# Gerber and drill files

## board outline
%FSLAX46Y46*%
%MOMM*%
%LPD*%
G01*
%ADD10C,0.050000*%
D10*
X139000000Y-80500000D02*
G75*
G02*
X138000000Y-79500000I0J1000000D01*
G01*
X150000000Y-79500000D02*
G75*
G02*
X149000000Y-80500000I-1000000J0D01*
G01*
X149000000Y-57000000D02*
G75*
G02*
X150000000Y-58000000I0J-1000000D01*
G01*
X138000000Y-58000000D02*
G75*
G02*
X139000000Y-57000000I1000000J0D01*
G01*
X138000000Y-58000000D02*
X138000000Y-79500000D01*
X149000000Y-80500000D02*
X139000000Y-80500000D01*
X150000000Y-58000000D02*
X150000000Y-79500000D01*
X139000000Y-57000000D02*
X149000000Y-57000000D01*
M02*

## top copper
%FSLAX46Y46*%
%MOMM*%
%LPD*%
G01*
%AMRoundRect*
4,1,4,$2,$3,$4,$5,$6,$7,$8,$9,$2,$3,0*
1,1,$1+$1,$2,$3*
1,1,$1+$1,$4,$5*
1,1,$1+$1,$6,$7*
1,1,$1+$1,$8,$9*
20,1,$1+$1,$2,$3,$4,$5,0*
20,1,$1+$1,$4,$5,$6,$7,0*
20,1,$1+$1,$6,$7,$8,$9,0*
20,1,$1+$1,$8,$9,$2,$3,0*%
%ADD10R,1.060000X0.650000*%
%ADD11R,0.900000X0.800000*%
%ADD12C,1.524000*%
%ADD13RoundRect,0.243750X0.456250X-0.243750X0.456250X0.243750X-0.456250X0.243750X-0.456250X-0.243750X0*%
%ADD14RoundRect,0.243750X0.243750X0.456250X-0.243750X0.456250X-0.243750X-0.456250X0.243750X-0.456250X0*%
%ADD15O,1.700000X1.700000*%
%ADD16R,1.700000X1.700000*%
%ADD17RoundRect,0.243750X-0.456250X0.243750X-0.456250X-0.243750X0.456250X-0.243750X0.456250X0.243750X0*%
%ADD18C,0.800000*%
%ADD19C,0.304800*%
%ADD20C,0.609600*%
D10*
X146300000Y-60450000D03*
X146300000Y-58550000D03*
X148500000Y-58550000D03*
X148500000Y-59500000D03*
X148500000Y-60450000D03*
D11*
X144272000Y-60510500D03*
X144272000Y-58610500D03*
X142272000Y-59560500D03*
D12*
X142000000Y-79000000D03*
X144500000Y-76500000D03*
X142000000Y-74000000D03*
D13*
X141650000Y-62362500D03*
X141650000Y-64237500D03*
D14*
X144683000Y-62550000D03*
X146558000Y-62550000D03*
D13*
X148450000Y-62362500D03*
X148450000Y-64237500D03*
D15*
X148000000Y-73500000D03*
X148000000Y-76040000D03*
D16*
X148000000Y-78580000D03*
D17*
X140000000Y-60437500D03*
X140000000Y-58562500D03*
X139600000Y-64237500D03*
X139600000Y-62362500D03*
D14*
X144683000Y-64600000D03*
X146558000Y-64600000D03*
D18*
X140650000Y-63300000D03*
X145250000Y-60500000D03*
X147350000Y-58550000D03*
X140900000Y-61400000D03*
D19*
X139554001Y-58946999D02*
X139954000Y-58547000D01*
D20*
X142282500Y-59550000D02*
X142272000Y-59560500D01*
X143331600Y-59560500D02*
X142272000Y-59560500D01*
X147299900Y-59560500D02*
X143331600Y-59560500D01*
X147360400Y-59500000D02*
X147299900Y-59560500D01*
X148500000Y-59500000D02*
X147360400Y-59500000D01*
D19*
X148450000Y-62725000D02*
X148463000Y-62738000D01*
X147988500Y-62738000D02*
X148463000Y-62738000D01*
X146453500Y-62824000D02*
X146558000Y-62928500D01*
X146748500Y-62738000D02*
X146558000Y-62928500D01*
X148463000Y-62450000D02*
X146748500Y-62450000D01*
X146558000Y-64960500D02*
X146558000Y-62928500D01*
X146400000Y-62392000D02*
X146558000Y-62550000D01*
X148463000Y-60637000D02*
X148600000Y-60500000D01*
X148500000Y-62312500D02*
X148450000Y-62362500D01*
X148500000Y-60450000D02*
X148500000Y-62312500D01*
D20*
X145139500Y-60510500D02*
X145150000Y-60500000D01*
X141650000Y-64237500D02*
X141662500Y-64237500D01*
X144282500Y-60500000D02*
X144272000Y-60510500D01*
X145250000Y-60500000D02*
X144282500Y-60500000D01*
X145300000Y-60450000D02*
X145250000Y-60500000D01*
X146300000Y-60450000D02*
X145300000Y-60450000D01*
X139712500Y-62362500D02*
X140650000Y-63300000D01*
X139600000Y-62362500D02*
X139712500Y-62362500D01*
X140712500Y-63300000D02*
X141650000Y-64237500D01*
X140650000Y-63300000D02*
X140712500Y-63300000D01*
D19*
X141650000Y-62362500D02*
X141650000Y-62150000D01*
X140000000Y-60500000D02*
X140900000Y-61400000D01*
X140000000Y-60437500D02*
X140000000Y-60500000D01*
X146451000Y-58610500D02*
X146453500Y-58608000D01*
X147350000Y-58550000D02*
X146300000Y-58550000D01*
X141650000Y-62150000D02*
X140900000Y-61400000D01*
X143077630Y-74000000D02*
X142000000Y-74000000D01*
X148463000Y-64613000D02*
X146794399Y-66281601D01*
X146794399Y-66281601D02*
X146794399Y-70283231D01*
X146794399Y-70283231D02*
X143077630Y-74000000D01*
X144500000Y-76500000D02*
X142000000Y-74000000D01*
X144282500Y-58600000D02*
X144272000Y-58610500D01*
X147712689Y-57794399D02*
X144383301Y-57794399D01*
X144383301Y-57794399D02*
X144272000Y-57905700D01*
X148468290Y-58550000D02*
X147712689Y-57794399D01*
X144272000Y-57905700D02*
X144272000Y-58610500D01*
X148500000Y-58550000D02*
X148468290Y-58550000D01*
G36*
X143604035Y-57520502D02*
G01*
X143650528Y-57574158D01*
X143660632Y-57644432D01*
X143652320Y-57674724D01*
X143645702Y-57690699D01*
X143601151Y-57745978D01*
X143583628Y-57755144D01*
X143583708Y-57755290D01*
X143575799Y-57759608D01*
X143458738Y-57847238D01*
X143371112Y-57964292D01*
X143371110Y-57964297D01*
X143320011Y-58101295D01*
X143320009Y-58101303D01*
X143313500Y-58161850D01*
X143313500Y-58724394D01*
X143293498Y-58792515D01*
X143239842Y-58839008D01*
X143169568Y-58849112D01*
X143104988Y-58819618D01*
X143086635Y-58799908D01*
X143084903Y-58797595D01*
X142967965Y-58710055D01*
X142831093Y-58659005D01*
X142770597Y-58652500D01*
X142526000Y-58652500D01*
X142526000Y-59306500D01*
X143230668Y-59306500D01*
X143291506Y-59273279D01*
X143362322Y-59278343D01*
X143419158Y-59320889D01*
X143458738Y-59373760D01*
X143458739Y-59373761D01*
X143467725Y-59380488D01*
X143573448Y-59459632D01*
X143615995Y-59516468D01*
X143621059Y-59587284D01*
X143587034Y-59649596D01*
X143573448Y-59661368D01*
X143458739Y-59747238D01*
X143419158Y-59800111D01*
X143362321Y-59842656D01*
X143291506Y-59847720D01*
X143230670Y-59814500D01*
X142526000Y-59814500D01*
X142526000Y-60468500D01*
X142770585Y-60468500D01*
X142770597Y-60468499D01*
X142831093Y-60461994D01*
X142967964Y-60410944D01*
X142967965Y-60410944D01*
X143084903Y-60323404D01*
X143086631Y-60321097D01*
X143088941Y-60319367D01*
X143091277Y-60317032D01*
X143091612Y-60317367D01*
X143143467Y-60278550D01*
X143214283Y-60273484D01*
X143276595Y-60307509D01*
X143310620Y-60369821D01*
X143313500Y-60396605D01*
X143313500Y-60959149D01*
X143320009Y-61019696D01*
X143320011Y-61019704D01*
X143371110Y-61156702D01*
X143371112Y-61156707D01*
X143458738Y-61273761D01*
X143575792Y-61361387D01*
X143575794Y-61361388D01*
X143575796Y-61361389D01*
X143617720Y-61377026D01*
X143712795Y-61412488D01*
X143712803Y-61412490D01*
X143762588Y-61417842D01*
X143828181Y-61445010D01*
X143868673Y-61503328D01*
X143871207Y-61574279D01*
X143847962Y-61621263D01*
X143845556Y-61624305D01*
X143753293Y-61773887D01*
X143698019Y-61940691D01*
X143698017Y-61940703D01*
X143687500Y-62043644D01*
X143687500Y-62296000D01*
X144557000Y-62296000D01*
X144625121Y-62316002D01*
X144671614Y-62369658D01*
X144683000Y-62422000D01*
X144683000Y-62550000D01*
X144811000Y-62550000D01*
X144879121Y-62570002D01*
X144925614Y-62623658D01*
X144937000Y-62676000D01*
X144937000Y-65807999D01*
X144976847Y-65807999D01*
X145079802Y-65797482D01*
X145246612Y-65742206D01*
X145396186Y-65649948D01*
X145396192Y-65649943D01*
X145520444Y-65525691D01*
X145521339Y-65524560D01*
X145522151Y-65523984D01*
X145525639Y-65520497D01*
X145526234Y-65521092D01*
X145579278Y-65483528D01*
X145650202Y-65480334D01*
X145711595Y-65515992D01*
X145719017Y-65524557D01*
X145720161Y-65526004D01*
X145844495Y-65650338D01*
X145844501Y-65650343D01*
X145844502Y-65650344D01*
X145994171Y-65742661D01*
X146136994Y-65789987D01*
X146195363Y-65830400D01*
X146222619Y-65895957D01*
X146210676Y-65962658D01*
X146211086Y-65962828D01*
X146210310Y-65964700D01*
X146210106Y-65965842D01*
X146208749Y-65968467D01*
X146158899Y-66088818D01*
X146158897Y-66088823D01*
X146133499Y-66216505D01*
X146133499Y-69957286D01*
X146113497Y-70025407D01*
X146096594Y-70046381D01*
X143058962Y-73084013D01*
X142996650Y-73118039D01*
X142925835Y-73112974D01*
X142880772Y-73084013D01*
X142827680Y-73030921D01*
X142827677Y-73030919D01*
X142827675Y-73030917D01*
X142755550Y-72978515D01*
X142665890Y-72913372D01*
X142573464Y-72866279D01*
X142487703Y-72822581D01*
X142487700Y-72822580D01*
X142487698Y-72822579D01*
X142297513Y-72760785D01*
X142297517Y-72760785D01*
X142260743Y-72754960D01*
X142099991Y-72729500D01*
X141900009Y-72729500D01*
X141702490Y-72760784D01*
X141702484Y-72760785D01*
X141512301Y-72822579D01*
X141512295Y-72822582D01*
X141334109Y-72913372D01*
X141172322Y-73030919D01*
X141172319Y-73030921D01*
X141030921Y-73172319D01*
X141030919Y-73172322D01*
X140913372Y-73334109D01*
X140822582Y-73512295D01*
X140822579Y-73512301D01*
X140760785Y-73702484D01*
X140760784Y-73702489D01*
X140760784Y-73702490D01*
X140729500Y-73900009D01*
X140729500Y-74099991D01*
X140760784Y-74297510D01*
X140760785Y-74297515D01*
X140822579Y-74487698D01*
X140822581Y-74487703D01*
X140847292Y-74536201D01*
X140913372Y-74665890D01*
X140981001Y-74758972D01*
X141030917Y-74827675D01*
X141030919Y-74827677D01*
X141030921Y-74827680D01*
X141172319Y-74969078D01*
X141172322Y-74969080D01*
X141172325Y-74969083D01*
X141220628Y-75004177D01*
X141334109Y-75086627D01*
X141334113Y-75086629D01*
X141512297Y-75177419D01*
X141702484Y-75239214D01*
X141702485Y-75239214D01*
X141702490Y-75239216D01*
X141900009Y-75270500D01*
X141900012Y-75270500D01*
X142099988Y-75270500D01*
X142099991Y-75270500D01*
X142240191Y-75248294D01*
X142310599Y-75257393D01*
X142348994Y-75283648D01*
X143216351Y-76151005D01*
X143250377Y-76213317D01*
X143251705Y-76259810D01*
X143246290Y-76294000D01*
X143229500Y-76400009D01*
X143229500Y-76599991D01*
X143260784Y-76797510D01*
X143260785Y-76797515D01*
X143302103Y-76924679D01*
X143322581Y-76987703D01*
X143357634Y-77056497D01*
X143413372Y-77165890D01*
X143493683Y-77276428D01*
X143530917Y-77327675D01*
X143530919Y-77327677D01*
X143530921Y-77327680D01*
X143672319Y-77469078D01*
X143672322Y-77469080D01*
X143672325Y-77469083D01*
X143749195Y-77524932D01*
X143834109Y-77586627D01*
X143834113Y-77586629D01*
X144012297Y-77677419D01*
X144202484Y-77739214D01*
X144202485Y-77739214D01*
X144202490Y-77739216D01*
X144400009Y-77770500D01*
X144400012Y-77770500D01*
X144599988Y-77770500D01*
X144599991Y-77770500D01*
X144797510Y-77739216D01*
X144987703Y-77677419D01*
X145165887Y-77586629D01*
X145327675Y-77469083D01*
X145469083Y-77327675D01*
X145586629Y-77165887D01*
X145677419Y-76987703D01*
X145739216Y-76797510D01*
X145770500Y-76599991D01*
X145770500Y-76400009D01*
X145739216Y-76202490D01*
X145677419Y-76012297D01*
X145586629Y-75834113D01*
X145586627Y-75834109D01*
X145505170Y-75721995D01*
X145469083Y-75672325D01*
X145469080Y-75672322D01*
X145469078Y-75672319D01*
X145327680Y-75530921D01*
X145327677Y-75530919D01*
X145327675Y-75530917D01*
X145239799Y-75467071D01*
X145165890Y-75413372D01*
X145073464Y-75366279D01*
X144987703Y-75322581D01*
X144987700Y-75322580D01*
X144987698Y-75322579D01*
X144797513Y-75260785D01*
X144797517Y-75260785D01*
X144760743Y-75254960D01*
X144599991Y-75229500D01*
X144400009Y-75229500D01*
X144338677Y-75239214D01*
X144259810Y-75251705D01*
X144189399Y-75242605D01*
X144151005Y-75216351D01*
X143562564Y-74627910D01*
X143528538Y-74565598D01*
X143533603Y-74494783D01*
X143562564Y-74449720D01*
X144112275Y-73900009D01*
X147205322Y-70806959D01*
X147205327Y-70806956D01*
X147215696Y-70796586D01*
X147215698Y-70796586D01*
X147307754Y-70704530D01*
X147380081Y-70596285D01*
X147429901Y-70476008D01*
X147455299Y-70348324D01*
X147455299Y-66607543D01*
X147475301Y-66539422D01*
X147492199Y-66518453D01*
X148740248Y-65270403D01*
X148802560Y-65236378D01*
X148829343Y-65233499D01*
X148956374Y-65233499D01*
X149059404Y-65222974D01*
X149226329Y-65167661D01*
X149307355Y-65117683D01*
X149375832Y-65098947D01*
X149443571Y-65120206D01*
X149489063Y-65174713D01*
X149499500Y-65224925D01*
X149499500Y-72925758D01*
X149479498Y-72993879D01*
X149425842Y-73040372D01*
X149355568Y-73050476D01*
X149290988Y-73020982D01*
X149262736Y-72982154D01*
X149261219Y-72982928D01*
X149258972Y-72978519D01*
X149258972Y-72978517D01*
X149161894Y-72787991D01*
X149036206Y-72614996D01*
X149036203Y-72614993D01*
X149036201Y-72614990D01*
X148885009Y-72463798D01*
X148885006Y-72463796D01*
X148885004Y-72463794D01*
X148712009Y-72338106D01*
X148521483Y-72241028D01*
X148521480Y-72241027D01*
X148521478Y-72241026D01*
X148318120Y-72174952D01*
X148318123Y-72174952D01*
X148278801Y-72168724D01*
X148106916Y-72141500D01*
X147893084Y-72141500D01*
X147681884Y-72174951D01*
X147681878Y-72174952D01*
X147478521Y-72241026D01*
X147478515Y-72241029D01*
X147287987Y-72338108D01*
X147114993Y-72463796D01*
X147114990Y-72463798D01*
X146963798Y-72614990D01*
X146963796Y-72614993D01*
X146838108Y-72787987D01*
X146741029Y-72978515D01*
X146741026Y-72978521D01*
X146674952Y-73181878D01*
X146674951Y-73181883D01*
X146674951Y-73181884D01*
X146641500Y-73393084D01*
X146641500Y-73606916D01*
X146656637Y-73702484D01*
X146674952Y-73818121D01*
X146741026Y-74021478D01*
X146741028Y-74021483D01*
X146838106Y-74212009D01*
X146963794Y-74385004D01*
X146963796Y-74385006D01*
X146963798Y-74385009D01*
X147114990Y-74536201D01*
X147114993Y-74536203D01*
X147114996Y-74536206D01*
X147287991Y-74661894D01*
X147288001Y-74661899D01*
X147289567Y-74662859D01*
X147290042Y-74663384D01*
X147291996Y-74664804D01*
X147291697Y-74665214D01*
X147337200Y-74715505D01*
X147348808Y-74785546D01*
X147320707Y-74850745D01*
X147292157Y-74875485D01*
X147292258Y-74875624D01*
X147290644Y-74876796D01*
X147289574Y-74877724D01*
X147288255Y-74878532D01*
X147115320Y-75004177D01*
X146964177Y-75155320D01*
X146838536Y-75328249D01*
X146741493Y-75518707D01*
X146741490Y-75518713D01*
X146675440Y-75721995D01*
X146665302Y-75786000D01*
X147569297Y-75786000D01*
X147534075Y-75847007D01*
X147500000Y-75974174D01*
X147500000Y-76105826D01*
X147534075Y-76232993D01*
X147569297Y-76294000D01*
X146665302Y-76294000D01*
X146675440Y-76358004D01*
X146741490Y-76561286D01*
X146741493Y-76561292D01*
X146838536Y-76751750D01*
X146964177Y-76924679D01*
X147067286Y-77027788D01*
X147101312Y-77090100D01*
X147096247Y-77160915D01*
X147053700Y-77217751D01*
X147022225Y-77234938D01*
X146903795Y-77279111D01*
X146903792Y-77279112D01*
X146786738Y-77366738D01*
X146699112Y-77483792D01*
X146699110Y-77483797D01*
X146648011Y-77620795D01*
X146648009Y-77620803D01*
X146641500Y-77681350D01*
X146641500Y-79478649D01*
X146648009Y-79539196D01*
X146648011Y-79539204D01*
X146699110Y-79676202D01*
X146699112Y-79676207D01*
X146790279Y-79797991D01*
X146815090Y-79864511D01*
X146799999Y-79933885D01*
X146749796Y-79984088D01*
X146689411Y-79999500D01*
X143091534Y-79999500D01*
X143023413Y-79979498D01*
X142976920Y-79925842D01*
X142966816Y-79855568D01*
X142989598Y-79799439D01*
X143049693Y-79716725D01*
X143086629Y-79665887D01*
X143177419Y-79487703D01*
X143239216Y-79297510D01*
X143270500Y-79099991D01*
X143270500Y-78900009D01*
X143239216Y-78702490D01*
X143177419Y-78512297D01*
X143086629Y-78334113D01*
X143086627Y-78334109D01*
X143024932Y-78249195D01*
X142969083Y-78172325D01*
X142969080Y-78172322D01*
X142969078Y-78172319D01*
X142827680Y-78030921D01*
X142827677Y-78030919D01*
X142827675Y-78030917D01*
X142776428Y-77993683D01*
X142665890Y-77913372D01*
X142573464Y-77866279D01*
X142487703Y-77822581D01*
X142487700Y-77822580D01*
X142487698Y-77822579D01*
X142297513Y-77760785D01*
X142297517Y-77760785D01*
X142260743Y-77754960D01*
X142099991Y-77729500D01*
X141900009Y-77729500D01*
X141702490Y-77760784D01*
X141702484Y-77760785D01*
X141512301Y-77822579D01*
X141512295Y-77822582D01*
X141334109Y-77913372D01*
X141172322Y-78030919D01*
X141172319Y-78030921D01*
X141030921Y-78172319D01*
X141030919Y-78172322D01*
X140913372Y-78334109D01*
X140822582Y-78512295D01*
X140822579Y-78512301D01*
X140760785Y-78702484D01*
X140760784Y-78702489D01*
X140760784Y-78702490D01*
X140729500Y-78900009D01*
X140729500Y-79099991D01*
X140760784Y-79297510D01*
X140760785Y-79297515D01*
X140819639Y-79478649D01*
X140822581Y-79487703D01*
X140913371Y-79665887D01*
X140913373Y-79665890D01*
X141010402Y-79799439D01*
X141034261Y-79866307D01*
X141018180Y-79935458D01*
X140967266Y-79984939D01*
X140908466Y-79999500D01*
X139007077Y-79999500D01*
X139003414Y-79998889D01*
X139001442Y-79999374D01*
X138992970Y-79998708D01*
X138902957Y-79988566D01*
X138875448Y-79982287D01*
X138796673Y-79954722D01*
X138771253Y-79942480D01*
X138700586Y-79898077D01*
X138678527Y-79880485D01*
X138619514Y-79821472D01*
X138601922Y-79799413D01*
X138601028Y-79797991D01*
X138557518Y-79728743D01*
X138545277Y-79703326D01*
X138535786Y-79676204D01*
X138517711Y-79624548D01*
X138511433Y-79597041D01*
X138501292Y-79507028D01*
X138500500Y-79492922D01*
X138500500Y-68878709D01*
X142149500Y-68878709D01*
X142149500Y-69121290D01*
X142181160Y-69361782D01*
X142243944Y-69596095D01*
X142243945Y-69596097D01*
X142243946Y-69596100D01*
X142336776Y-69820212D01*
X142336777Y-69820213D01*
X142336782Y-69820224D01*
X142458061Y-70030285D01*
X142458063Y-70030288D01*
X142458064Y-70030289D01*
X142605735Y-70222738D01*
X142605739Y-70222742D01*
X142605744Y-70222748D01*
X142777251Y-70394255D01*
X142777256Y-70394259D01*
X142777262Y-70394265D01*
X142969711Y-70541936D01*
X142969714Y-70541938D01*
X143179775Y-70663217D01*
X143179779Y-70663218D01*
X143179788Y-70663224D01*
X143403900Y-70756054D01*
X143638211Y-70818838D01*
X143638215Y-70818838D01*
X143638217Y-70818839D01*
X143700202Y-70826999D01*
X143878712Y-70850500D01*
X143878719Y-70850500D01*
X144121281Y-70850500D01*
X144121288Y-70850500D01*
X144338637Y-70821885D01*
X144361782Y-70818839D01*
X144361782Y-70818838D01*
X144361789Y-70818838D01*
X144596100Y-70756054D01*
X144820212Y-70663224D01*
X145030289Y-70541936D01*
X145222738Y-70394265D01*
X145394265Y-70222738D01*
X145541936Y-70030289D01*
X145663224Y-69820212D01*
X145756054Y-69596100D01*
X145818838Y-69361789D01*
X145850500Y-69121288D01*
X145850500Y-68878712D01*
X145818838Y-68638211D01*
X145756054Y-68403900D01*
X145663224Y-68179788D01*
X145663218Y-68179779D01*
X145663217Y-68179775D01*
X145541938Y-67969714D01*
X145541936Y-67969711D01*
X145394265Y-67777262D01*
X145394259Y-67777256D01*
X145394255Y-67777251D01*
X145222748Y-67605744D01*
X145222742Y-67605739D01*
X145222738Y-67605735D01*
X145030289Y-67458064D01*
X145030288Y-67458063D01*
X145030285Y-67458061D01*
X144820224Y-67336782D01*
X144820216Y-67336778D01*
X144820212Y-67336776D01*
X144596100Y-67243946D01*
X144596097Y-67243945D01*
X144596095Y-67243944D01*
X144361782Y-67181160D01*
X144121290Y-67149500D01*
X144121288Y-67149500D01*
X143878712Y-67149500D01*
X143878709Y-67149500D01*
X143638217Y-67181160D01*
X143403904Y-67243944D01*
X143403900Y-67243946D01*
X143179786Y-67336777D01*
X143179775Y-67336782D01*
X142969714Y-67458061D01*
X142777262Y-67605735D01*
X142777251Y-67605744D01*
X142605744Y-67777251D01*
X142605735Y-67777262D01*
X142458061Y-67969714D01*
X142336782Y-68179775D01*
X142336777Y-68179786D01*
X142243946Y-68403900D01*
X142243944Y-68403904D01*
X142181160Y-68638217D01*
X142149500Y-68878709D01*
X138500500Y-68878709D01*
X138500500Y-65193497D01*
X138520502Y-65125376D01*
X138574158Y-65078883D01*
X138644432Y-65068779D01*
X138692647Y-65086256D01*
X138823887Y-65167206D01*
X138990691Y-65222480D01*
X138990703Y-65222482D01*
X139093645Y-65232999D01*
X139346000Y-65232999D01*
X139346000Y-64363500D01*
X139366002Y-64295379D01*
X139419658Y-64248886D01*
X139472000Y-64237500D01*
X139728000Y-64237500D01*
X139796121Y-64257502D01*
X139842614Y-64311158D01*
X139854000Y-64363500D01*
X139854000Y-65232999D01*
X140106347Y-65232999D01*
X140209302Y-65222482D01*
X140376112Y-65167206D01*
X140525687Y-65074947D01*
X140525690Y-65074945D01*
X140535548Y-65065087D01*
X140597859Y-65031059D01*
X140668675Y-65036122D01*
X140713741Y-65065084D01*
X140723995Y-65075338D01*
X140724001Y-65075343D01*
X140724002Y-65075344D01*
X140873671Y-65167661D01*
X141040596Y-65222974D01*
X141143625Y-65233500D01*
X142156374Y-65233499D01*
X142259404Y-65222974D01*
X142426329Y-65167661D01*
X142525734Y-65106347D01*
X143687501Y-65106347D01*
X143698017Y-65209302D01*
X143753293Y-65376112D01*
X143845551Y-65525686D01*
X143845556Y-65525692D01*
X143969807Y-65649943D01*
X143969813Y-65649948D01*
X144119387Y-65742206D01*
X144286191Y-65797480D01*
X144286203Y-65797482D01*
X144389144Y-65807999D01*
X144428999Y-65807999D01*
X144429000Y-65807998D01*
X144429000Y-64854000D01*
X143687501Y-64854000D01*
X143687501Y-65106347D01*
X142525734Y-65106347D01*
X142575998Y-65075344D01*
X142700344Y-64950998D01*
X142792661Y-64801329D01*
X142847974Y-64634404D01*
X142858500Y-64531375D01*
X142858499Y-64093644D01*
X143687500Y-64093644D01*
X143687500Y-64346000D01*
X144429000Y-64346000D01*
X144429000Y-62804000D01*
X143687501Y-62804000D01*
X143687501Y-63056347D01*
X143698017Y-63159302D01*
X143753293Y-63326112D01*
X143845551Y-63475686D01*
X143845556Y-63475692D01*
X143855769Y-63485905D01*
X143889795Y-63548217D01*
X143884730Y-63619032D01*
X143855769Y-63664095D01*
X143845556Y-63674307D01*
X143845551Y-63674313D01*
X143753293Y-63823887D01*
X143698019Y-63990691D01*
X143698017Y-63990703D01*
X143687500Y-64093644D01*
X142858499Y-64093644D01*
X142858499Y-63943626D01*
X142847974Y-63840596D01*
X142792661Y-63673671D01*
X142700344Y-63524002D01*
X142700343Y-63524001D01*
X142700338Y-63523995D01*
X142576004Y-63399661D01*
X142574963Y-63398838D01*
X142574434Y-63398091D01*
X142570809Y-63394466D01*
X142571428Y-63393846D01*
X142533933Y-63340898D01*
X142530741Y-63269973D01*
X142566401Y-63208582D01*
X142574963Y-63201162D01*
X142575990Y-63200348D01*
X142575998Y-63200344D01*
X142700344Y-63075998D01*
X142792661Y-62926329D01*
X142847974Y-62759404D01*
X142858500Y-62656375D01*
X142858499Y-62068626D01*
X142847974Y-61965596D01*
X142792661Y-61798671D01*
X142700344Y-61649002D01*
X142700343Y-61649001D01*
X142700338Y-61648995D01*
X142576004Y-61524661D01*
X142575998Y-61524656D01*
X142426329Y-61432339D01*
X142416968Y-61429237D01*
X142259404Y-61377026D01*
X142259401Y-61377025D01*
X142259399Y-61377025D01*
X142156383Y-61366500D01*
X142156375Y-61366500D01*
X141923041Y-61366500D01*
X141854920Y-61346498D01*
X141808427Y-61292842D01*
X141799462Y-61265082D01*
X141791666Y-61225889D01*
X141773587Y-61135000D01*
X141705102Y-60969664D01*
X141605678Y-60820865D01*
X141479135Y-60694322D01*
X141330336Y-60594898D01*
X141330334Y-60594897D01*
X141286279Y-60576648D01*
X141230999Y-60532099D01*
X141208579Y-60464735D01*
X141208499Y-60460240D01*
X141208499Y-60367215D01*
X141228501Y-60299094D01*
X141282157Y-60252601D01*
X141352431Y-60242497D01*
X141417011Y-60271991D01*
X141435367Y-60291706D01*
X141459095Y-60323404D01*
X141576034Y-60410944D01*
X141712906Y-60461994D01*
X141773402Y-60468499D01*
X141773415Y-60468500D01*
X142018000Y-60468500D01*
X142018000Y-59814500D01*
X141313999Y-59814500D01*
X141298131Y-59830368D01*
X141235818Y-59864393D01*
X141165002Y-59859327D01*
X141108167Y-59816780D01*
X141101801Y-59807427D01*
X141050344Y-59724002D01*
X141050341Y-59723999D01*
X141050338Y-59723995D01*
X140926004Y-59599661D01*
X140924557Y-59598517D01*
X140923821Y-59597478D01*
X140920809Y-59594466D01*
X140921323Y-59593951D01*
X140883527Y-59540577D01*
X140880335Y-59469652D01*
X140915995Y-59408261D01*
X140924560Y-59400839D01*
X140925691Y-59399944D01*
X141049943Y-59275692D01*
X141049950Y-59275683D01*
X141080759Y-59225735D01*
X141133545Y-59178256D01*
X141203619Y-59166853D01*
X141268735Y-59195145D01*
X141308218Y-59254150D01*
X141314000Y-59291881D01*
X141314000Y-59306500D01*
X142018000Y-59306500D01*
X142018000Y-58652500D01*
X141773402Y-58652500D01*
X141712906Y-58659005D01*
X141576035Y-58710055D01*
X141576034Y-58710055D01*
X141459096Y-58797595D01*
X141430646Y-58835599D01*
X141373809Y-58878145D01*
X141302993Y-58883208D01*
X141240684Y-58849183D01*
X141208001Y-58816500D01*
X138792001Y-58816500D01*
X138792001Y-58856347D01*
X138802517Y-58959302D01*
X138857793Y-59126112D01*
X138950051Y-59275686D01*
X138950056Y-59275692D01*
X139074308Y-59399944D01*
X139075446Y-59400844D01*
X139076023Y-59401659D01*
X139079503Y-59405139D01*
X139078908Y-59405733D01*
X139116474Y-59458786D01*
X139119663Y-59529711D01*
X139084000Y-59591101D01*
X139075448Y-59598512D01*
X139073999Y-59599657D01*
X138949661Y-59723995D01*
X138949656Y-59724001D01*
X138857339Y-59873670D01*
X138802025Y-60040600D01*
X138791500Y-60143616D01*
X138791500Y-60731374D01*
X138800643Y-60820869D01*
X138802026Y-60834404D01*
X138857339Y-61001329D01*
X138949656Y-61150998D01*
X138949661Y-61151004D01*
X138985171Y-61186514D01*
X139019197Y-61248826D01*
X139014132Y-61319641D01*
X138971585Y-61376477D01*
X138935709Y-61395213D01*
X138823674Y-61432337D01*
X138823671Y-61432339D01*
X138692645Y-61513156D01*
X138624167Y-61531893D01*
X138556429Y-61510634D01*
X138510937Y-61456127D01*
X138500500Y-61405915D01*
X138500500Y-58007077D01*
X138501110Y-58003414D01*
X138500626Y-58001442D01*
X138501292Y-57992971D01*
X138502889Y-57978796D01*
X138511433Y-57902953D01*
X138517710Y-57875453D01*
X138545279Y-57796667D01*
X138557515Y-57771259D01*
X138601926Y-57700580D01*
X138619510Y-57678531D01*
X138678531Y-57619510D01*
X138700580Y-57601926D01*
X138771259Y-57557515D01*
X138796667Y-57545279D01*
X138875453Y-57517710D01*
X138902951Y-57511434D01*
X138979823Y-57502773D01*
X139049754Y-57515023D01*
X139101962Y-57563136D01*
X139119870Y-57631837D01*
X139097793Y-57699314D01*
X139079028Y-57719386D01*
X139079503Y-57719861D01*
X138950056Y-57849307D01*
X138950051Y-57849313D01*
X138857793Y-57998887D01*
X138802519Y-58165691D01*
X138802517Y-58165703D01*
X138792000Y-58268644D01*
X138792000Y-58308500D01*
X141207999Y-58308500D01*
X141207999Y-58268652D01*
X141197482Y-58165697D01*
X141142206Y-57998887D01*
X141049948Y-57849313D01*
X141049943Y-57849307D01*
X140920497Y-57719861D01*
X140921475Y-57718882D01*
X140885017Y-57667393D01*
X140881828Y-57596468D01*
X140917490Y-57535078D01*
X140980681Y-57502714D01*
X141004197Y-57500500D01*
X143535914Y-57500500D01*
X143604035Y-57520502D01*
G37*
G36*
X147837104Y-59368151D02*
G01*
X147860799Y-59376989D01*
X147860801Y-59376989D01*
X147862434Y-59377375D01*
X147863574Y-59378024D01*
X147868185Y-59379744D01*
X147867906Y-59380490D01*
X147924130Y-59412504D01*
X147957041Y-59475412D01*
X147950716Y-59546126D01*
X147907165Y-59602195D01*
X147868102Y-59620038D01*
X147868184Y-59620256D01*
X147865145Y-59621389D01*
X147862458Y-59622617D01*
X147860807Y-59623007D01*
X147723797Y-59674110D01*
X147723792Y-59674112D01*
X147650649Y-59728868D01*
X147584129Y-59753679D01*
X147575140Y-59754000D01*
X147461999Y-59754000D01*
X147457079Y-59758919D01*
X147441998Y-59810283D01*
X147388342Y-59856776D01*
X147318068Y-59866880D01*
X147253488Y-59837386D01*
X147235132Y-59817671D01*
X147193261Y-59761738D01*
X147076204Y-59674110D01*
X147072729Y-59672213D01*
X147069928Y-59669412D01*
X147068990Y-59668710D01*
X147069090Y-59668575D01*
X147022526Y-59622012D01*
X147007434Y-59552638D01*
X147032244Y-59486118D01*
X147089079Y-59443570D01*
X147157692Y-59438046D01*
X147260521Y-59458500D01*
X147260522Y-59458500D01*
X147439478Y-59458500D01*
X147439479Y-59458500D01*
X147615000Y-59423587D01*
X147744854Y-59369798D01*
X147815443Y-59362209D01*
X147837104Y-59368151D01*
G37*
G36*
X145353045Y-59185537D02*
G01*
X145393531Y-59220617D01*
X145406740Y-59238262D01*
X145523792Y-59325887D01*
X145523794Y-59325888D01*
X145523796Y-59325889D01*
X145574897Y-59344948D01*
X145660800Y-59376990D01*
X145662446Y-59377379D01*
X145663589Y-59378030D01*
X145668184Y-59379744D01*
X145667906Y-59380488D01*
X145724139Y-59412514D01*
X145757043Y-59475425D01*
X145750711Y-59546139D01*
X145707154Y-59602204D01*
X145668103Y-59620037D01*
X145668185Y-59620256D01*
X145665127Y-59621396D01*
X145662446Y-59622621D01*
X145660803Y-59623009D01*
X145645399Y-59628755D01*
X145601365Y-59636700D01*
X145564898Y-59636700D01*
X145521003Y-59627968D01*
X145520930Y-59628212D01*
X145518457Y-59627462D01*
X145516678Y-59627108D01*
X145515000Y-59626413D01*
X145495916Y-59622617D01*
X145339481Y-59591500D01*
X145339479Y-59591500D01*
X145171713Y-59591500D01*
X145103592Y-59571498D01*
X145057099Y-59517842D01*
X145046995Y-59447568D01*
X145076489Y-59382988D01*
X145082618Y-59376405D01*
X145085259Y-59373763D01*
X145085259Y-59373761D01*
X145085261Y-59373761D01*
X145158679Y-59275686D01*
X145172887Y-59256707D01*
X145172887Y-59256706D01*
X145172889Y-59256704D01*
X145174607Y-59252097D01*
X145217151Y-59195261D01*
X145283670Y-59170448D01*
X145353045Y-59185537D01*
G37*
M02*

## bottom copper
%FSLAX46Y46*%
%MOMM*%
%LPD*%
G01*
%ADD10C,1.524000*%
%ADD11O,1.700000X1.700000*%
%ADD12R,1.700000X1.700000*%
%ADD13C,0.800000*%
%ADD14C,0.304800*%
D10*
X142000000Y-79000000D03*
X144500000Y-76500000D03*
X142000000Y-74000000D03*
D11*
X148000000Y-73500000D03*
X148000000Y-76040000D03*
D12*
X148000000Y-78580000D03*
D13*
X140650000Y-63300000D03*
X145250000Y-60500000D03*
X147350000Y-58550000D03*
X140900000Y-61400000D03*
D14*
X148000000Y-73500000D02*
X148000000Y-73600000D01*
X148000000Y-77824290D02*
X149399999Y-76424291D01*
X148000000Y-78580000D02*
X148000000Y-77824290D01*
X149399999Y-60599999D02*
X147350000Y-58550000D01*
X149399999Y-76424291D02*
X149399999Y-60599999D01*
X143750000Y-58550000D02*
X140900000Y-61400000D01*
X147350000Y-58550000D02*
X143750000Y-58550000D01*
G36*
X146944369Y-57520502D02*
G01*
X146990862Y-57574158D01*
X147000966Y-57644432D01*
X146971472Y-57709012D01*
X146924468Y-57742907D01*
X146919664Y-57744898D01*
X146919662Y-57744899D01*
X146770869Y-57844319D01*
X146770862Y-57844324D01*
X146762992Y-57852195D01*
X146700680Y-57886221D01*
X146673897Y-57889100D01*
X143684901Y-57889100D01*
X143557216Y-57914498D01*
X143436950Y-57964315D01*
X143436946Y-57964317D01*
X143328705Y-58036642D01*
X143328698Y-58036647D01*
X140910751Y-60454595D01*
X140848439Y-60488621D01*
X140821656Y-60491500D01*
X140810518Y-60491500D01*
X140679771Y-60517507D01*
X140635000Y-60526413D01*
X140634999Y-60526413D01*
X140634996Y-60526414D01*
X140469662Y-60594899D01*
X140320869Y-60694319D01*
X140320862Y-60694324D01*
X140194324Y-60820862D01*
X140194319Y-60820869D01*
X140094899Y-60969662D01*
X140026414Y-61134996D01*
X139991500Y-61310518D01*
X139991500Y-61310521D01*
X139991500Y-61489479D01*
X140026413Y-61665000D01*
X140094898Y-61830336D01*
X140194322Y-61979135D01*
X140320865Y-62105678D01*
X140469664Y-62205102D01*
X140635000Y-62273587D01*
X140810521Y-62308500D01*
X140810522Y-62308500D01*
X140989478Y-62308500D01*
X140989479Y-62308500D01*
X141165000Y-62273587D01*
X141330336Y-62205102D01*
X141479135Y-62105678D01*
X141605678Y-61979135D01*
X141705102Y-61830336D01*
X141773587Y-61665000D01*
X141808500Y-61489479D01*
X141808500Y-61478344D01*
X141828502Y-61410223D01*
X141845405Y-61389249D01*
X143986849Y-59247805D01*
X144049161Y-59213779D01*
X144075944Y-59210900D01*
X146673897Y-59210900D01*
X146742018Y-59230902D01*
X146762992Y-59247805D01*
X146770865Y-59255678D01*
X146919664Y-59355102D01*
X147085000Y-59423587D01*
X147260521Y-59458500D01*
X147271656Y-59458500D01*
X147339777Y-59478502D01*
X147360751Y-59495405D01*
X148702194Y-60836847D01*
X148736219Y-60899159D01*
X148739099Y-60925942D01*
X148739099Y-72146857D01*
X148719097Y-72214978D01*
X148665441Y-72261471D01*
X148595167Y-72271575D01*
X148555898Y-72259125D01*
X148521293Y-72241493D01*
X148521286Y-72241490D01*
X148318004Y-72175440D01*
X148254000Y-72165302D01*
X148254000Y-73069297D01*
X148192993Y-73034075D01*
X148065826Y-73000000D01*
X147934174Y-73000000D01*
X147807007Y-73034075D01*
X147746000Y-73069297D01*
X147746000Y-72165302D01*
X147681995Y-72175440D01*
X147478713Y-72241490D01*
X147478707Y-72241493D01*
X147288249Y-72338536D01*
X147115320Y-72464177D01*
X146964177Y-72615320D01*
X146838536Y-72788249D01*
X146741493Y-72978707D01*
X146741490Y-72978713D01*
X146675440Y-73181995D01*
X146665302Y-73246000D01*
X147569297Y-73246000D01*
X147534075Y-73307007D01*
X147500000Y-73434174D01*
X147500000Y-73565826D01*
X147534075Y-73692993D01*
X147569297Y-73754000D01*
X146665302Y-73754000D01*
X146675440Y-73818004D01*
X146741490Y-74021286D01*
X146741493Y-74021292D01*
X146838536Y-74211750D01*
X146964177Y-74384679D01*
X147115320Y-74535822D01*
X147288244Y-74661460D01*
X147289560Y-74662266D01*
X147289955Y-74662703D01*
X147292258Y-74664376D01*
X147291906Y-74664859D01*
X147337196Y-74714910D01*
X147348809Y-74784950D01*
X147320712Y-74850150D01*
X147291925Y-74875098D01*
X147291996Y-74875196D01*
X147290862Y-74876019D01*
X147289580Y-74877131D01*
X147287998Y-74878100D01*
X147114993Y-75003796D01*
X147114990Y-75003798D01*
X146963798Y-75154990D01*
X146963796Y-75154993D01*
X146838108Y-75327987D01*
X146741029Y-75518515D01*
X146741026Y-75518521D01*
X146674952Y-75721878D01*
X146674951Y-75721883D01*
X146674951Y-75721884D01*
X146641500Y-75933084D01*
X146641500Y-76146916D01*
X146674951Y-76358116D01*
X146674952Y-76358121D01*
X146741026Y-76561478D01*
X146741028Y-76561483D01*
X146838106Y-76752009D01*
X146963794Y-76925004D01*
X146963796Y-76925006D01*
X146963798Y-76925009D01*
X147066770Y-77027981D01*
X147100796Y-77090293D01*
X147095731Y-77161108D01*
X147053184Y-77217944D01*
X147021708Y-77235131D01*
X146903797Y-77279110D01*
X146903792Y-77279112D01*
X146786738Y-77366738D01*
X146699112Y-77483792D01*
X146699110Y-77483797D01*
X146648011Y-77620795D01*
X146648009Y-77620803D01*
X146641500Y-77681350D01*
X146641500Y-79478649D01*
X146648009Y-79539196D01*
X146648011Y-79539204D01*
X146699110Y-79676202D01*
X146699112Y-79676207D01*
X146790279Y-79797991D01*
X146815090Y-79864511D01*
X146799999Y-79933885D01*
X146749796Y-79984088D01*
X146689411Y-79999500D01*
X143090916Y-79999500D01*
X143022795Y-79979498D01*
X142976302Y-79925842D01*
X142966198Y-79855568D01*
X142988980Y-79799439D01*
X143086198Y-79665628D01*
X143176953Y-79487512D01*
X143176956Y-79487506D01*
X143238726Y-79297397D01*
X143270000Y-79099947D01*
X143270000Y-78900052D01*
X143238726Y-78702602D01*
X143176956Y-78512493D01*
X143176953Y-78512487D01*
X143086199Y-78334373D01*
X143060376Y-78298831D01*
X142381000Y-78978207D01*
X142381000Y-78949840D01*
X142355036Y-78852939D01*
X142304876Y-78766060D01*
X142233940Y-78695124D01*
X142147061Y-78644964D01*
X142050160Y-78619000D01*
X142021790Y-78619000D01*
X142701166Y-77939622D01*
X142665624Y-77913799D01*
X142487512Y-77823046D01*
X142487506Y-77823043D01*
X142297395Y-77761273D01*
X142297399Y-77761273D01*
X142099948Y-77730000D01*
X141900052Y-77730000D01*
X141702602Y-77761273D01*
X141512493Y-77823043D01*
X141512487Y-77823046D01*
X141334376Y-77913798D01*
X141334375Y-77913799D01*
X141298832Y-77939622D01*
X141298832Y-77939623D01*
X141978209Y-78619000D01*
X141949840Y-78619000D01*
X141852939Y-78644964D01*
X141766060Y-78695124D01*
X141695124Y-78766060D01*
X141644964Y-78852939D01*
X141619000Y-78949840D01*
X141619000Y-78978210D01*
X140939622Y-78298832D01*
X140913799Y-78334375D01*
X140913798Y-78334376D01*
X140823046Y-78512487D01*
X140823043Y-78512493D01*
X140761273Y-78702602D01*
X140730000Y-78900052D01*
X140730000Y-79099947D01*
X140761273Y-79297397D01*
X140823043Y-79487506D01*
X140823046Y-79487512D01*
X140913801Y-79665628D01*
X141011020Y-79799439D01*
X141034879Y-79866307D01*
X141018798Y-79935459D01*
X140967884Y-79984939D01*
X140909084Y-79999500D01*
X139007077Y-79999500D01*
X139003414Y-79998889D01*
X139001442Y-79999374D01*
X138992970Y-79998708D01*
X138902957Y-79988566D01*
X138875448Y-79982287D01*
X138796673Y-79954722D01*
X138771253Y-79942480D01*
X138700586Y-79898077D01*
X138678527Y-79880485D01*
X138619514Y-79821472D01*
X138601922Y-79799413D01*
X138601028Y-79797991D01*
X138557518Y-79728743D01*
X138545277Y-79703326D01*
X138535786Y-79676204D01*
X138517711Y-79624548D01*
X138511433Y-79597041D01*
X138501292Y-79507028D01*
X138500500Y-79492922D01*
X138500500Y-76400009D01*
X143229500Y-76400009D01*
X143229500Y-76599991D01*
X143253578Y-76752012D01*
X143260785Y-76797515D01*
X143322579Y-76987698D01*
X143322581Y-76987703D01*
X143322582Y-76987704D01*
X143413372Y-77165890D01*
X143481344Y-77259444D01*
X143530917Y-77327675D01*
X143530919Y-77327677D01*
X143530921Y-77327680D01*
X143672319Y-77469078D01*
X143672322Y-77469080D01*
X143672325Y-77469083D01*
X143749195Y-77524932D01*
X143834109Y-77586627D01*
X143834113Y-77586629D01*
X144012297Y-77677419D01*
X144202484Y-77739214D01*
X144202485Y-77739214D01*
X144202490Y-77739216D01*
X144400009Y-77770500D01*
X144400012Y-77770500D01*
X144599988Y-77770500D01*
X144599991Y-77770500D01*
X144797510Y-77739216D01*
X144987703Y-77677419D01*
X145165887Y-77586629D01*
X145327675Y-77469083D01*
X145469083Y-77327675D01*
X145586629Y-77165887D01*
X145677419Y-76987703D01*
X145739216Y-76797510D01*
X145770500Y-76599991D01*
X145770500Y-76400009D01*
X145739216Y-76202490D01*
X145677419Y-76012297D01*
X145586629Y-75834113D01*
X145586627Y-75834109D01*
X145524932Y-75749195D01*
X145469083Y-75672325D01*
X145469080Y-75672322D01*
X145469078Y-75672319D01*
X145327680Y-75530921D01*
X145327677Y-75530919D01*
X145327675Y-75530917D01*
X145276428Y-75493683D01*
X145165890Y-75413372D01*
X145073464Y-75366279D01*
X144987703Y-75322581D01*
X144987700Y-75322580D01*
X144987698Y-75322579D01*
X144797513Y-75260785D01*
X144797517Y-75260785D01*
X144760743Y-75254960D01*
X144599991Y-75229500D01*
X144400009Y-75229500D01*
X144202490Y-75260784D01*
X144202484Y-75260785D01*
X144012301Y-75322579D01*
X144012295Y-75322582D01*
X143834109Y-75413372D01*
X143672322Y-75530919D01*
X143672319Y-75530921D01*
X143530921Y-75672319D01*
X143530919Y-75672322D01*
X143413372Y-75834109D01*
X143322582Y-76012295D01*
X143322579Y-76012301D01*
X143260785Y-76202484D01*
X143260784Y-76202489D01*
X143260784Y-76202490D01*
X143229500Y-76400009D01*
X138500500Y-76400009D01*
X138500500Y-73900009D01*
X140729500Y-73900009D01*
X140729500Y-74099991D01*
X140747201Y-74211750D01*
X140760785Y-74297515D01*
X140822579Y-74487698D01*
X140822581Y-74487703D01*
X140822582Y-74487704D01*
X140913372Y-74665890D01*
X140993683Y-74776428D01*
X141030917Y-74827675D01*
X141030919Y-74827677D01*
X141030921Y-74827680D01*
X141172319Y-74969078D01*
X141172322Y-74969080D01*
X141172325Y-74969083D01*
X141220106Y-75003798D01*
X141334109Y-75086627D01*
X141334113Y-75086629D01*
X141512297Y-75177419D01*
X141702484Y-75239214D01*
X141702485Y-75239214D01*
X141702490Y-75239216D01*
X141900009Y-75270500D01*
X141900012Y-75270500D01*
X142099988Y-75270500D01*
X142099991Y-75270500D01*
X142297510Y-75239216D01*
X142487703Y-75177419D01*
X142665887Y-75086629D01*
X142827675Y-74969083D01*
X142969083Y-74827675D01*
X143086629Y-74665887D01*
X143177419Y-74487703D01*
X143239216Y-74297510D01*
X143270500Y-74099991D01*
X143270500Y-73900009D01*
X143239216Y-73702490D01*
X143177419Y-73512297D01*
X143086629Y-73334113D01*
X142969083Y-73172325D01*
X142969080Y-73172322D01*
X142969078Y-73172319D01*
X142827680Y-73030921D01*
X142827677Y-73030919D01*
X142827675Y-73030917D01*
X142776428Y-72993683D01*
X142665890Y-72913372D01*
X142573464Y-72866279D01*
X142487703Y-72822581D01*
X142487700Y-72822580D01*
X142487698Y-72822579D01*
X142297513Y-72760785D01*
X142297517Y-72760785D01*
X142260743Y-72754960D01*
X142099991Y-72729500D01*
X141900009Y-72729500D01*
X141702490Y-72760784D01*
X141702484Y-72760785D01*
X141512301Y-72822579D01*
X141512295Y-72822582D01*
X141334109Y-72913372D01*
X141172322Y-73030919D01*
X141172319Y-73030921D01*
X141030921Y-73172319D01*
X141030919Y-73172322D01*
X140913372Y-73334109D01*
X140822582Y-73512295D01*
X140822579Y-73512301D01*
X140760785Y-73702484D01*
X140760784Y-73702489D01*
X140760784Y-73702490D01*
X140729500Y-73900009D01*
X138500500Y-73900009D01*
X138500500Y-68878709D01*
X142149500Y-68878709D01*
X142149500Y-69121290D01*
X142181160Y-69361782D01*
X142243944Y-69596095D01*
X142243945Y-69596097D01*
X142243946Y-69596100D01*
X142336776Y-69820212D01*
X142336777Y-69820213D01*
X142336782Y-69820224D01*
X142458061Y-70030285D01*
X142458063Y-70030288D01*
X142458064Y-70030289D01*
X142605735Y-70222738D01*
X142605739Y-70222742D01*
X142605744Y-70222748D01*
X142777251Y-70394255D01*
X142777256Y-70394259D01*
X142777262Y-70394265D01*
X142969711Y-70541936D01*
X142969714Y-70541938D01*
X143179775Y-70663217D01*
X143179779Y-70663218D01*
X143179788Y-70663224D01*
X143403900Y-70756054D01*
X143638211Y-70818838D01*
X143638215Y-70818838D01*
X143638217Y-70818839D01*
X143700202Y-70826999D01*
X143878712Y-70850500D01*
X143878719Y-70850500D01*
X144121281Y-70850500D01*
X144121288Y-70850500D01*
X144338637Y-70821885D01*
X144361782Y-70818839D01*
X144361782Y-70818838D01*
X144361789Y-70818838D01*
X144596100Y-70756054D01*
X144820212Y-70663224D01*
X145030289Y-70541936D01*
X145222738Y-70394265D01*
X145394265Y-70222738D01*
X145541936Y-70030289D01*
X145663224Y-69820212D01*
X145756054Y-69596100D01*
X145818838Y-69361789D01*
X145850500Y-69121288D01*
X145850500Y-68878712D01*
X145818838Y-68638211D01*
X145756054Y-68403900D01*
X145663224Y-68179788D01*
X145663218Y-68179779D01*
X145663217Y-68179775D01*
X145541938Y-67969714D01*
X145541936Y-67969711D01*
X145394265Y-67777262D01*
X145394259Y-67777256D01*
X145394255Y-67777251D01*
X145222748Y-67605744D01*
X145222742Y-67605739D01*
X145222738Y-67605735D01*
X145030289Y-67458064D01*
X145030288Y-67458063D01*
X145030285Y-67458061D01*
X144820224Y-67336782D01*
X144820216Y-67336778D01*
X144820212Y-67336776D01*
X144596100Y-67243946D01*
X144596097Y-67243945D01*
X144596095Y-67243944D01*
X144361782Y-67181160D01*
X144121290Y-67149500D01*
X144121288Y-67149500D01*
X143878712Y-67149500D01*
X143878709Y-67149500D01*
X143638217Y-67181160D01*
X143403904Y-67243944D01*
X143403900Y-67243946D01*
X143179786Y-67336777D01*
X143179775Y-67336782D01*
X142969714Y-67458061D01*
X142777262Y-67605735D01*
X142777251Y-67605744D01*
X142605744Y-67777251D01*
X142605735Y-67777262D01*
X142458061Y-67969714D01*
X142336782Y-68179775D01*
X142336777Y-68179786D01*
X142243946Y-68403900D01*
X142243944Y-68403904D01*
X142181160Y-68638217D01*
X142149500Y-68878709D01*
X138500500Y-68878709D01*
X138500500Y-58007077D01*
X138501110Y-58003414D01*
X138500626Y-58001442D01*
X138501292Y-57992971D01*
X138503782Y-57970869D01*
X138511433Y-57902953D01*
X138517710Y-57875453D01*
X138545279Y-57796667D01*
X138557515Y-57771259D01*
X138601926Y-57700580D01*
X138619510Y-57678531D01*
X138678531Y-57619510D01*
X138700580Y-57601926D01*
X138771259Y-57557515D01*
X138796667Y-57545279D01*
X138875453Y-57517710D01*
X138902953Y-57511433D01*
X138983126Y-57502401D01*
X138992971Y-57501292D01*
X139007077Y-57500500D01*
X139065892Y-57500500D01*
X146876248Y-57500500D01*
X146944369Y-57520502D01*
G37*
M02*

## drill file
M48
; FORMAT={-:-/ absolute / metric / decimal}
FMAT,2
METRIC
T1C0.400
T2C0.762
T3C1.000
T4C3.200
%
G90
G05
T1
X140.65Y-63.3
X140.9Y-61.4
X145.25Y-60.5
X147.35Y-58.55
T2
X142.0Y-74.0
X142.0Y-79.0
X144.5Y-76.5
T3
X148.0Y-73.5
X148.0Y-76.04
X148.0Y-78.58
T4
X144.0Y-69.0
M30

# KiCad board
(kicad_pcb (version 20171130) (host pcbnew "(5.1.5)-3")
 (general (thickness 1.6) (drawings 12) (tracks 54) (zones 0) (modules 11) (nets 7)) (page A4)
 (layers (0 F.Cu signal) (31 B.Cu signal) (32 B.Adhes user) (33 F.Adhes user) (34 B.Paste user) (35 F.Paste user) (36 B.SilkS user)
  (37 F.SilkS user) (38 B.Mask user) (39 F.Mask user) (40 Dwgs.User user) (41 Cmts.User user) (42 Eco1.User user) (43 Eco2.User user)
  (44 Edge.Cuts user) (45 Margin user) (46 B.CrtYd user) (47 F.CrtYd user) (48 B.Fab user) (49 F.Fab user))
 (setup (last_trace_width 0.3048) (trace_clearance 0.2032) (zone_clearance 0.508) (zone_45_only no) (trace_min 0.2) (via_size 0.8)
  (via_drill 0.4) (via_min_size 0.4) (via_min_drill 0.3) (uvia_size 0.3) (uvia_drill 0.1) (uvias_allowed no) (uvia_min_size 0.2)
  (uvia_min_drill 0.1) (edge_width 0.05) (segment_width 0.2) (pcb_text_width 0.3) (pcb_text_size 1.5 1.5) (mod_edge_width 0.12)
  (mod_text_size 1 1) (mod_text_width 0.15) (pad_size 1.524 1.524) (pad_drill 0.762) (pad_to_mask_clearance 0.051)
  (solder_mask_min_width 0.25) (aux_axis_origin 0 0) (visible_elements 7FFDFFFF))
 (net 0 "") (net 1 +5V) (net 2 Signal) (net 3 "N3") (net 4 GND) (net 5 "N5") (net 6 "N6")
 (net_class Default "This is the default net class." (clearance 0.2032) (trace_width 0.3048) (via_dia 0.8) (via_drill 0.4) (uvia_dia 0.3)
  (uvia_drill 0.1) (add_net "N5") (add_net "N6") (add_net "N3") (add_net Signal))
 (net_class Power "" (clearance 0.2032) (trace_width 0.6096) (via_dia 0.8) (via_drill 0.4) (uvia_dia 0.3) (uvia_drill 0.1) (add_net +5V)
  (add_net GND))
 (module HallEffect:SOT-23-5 (layer F.Cu) (at 147.4 59.5 180)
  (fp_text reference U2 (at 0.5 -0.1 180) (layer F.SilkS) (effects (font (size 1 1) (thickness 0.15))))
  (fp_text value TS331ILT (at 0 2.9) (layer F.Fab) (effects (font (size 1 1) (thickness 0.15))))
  (pad 5 smd rect (at 1.1 -0.95 180) (size 1.06 0.65) (layers F.Cu F.Paste F.Mask) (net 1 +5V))
  (pad 4 smd rect (at 1.1 0.95 180) (size 1.06 0.65) (layers F.Cu F.Paste F.Mask) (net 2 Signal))
  (pad 3 smd rect (at -1.1 0.95 180) (size 1.06 0.65) (layers F.Cu F.Paste F.Mask) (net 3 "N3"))
  (pad 2 smd rect (at -1.1 0 180) (size 1.06 0.65) (layers F.Cu F.Paste F.Mask) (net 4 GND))
  (pad 1 smd rect (at -1.1 -0.95 180) (size 1.06 0.65) (layers F.Cu F.Paste F.Mask) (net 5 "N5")))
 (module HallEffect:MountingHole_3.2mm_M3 (layer F.Cu) (at 144 69)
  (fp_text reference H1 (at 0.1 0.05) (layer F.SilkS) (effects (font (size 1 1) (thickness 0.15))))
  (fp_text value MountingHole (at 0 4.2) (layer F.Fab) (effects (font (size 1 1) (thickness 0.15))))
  (pad 1 np_thru_hole circle (at 0 0) (size 3.2 3.2) (drill 3.2) (layers *.Cu *.Mask)))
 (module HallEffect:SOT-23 (layer F.Cu) (at 143.272 59.5605 180)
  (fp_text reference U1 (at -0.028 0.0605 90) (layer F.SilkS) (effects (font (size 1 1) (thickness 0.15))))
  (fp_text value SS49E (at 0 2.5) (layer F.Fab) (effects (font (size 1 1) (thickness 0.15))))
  (pad 1 smd rect (at -1 -0.95 180) (size 0.9 0.8) (layers F.Cu F.Paste F.Mask) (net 1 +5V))
  (pad 2 smd rect (at -1 0.95 180) (size 0.9 0.8) (layers F.Cu F.Paste F.Mask) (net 3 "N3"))
  (pad 3 smd rect (at 1 0 180) (size 0.9 0.8) (layers F.Cu F.Paste F.Mask) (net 4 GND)))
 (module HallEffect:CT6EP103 (layer F.Cu) (at 142 76.5 270)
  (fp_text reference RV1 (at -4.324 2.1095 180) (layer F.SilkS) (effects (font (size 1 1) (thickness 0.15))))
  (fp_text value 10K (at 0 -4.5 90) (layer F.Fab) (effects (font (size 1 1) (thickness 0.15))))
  (pad 3 thru_hole circle (at 2.5 0 270) (size 1.524 1.524) (drill 0.762) (layers *.Cu *.Mask) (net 1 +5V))
  (pad 2 thru_hole circle (at 0 -2.5 270) (size 1.524 1.524) (drill 0.762) (layers *.Cu *.Mask) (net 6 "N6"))
  (pad 1 thru_hole circle (at -2.5 0 270) (size 1.524 1.524) (drill 0.762) (layers *.Cu *.Mask) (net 6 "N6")))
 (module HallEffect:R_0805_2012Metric (layer F.Cu) (at 141.65 63.3 90)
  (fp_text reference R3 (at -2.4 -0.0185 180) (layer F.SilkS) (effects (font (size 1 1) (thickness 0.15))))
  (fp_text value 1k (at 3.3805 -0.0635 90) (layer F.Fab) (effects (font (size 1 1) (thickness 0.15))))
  (pad 2 smd roundrect (at 0.9375 0 90) (size 0.975 1.4) (layers F.Cu F.Paste F.Mask) (roundrect_rratio 0.25) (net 2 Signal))
  (pad 1 smd roundrect (at -0.9375 0 90) (size 0.975 1.4) (layers F.Cu F.Paste F.Mask) (roundrect_rratio 0.25) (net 1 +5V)))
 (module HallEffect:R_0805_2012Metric (layer F.Cu) (at 145.6205 62.55 180)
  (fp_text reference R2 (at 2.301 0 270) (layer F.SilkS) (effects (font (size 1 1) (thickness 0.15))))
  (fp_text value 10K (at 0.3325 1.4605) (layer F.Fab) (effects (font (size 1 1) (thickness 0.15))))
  (pad 2 smd roundrect (at 0.9375 0 180) (size 0.975 1.4) (layers F.Cu F.Paste F.Mask) (roundrect_rratio 0.25) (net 4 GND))
  (pad 1 smd roundrect (at -0.9375 0 180) (size 0.975 1.4) (layers F.Cu F.Paste F.Mask) (roundrect_rratio 0.25) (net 5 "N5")))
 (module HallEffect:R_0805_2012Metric (layer F.Cu) (at 148.45 63.3 90)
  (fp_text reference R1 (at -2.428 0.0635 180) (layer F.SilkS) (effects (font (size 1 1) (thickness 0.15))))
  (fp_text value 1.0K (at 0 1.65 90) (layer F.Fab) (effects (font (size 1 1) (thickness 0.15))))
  (pad 2 smd roundrect (at 0.9375 0 90) (size 0.975 1.4) (layers F.Cu F.Paste F.Mask) (roundrect_rratio 0.25) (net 5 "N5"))
  (pad 1 smd roundrect (at -0.9375 0 90) (size 0.975 1.4) (layers F.Cu F.Paste F.Mask) (roundrect_rratio 0.25) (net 6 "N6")))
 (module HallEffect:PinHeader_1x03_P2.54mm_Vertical (layer F.Cu) (at 148 78.58 180)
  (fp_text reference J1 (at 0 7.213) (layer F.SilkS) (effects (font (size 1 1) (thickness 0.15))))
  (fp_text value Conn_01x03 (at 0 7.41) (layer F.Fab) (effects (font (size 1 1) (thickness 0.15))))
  (pad 3 thru_hole oval (at 0 5.08 180) (size 1.7 1.7) (drill 1) (layers *.Cu *.Mask) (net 1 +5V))
  (pad 2 thru_hole oval (at 0 2.54 180) (size 1.7 1.7) (drill 1) (layers *.Cu *.Mask) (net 4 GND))
  (pad 1 thru_hole rect (at 0 0 180) (size 1.7 1.7) (drill 1) (layers *.Cu *.Mask) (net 2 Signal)))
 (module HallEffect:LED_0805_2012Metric (layer F.Cu) (at 140 59.5 270)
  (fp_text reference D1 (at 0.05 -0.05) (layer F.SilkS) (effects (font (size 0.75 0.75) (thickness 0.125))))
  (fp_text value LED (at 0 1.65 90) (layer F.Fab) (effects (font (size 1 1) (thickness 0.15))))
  (pad 2 smd roundrect (at 0.9375 0 270) (size 0.975 1.4) (layers F.Cu F.Paste F.Mask) (roundrect_rratio 0.25) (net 2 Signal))
  (pad 1 smd roundrect (at -0.9375 0 270) (size 0.975 1.4) (layers F.Cu F.Paste F.Mask) (roundrect_rratio 0.25) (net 4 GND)))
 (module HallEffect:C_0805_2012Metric (layer F.Cu) (at 139.6 63.3 270)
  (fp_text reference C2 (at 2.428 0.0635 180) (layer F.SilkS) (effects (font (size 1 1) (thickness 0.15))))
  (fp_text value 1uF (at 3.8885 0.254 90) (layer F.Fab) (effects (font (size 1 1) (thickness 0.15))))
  (pad 2 smd roundrect (at 0.9375 0 270) (size 0.975 1.4) (layers F.Cu F.Paste F.Mask) (roundrect_rratio 0.25) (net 4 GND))
  (pad 1 smd roundrect (at -0.9375 0 270) (size 0.975 1.4) (layers F.Cu F.Paste F.Mask) (roundrect_rratio 0.25) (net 1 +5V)))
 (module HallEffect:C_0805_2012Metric (layer F.Cu) (at 145.6205 64.6 180)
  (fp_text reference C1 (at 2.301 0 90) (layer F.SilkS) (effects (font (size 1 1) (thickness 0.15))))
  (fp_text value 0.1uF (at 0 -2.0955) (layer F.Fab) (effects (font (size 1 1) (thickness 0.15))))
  (pad 2 smd roundrect (at 0.9375 0 180) (size 0.975 1.4) (layers F.Cu F.Paste F.Mask) (roundrect_rratio 0.25) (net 4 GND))
  (pad 1 smd roundrect (at -0.9375 0 180) (size 0.975 1.4) (layers F.Cu F.Paste F.Mask) (roundrect_rratio 0.25) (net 5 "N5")))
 (gr_arc (start 139 79.5) (end 138 79.5) (angle -90) (layer Edge.Cuts) (width 0.05))
 (gr_arc (start 149 79.5) (end 149 80.5) (angle -90) (layer Edge.Cuts) (width 0.05))
 (gr_arc (start 149 58) (end 150 58) (angle -90) (layer Edge.Cuts) (width 0.05))
 (gr_arc (start 139 58) (end 139 57) (angle -90) (layer Edge.Cuts) (width 0.05))
 (gr_line (start 138 58) (end 138 79.5) (layer Edge.Cuts) (width 0.05))
 (gr_line (start 149 80.5) (end 139 80.5) (layer Edge.Cuts) (width 0.05))
 (gr_line (start 150 58) (end 150 79.5) (layer Edge.Cuts) (width 0.05))
 (gr_line (start 139 57) (end 149 57) (layer Edge.Cuts) (width 0.05))
 (segment (start 139.554001 58.946999) (end 139.954 58.547) (width 0.3048) (layer F.Cu) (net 4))
 (segment (start 142.2825 59.55) (end 142.272 59.5605) (width 0.6096) (layer F.Cu) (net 4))
 (segment (start 143.3316 59.5605) (end 142.272 59.5605) (width 0.6096) (layer F.Cu) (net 4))
 (segment (start 147.2999 59.5605) (end 143.3316 59.5605) (width 0.6096) (layer F.Cu) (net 4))
 (segment (start 147.3604 59.5) (end 147.2999 59.5605) (width 0.6096) (layer F.Cu) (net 4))
 (segment (start 148.5 59.5) (end 147.3604 59.5) (width 0.6096) (layer F.Cu) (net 4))
 (segment (start 148.45 62.725) (end 148.463 62.738) (width 0.3048) (layer F.Cu) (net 5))
 (segment (start 147.9885 62.738) (end 148.463 62.738) (width 0.3048) (layer F.Cu) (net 5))
 (segment (start 146.4535 62.824) (end 146.558 62.9285) (width 0.3048) (layer F.Cu) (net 5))
 (segment (start 146.7485 62.738) (end 146.558 62.9285) (width 0.3048) (layer F.Cu) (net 5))
 (segment (start 148.463 62.45) (end 146.7485 62.45) (width 0.3048) (layer F.Cu) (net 5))
 (segment (start 146.558 64.9605) (end 146.558 62.9285) (width 0.3048) (layer F.Cu) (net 5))
 (segment (start 146.4 62.392) (end 146.558 62.55) (width 0.3048) (layer F.Cu) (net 5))
 (segment (start 148.463 60.637) (end 148.6 60.5) (width 0.3048) (layer F.Cu) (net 5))
 (segment (start 148.5 62.3125) (end 148.45 62.3625) (width 0.3048) (layer F.Cu) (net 5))
 (segment (start 148.5 60.45) (end 148.5 62.3125) (width 0.3048) (layer F.Cu) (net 5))
 (via (at 140.65 63.3) (size 0.8) (drill 0.4) (layers F.Cu B.Cu) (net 1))
 (via (at 145.25 60.5) (size 0.8) (drill 0.4) (layers F.Cu B.Cu) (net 1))
 (segment (start 145.1395 60.5105) (end 145.15 60.5) (width 0.6096) (layer F.Cu) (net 1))
 (segment (start 141.65 64.2375) (end 141.6625 64.2375) (width 0.6096) (layer F.Cu) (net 1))
 (segment (start 148 73.5) (end 148 73.6) (width 0.3048) (layer B.Cu) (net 1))
 (segment (start 144.2825 60.5) (end 144.272 60.5105) (width 0.6096) (layer F.Cu) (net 1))
 (segment (start 145.25 60.5) (end 144.2825 60.5) (width 0.6096) (layer F.Cu) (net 1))
 (segment (start 145.3 60.45) (end 145.25 60.5) (width 0.6096) (layer F.Cu) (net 1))
 (segment (start 146.3 60.45) (end 145.3 60.45) (width 0.6096) (layer F.Cu) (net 1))
 (segment (start 139.7125 62.3625) (end 140.65 63.3) (width 0.6096) (layer F.Cu) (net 1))
 (segment (start 139.6 62.3625) (end 139.7125 62.3625) (width 0.6096) (layer F.Cu) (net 1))
 (segment (start 140.7125 63.3) (end 141.65 64.2375) (width 0.6096) (layer F.Cu) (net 1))
 (segment (start 140.65 63.3) (end 140.7125 63.3) (width 0.6096) (layer F.Cu) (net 1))
 (via (at 147.35 58.55) (size 0.8) (drill 0.4) (layers F.Cu B.Cu) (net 2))
 (via (at 140.9 61.4) (size 0.8) (drill 0.4) (layers F.Cu B.Cu) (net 2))
 (segment (start 141.65 62.3625) (end 141.65 62.15) (width 0.3048) (layer F.Cu) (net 2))
 (segment (start 140 60.5) (end 140.9 61.4) (width 0.3048) (layer F.Cu) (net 2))
 (segment (start 140 60.4375) (end 140 60.5) (width 0.3048) (layer F.Cu) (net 2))
 (segment (start 148 77.82429) (end 149.399999 76.424291) (width 0.3048) (layer B.Cu) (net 2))
 (segment (start 148 78.58) (end 148 77.82429) (width 0.3048) (layer B.Cu) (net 2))
 (segment (start 146.451 58.6105) (end 146.4535 58.608) (width 0.3048) (layer F.Cu) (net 2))
 (segment (start 147.35 58.55) (end 146.3 58.55) (width 0.3048) (layer F.Cu) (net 2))
 (segment (start 141.65 62.15) (end 140.9 61.4) (width 0.3048) (layer F.Cu) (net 2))
 (segment (start 149.399999 60.599999) (end 147.35 58.55) (width 0.3048) (layer B.Cu) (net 2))
 (segment (start 149.399999 76.424291) (end 149.399999 60.599999) (width 0.3048) (layer B.Cu) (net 2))
 (segment (start 143.75 58.55) (end 140.9 61.4) (width 0.3048) (layer B.Cu) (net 2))
 (segment (start 147.35 58.55) (end 143.75 58.55) (width 0.3048) (layer B.Cu) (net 2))
 (segment (start 143.07763 74) (end 142 74) (width 0.3048) (layer F.Cu) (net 6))
 (segment (start 148.463 64.613) (end 146.794399 66.281601) (width 0.3048) (layer F.Cu) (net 6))
 (segment (start 146.794399 66.281601) (end 146.794399 70.283231) (width 0.3048) (layer F.Cu) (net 6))
 (segment (start 146.794399 70.283231) (end 143.07763 74) (width 0.3048) (layer F.Cu) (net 6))
 (segment (start 144.5 76.5) (end 142 74) (width 0.3048) (layer F.Cu) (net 6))
 (segment (start 144.2825 58.6) (end 144.272 58.6105) (width 0.3048) (layer F.Cu) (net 3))
 (segment (start 147.712689 57.794399) (end 144.383301 57.794399) (width 0.3048) (layer F.Cu) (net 3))
 (segment (start 144.383301 57.794399) (end 144.272 57.9057) (width 0.3048) (layer F.Cu) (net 3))
 (segment (start 148.46829 58.55) (end 147.712689 57.794399) (width 0.3048) (layer F.Cu) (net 3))
 (segment (start 144.272 57.9057) (end 144.272 58.6105) (width 0.3048) (layer F.Cu) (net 3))
 (segment (start 148.5 58.55) (end 148.46829 58.55) (width 0.3048) (layer F.Cu) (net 3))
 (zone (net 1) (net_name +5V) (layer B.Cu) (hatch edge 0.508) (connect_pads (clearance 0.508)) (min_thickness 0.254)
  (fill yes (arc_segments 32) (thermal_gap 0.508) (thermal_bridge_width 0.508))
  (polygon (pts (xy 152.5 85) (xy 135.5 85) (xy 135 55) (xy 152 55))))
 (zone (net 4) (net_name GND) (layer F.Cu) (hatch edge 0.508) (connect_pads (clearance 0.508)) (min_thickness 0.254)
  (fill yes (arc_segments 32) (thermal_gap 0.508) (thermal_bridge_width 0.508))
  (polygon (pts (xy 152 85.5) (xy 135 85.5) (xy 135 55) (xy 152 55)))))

